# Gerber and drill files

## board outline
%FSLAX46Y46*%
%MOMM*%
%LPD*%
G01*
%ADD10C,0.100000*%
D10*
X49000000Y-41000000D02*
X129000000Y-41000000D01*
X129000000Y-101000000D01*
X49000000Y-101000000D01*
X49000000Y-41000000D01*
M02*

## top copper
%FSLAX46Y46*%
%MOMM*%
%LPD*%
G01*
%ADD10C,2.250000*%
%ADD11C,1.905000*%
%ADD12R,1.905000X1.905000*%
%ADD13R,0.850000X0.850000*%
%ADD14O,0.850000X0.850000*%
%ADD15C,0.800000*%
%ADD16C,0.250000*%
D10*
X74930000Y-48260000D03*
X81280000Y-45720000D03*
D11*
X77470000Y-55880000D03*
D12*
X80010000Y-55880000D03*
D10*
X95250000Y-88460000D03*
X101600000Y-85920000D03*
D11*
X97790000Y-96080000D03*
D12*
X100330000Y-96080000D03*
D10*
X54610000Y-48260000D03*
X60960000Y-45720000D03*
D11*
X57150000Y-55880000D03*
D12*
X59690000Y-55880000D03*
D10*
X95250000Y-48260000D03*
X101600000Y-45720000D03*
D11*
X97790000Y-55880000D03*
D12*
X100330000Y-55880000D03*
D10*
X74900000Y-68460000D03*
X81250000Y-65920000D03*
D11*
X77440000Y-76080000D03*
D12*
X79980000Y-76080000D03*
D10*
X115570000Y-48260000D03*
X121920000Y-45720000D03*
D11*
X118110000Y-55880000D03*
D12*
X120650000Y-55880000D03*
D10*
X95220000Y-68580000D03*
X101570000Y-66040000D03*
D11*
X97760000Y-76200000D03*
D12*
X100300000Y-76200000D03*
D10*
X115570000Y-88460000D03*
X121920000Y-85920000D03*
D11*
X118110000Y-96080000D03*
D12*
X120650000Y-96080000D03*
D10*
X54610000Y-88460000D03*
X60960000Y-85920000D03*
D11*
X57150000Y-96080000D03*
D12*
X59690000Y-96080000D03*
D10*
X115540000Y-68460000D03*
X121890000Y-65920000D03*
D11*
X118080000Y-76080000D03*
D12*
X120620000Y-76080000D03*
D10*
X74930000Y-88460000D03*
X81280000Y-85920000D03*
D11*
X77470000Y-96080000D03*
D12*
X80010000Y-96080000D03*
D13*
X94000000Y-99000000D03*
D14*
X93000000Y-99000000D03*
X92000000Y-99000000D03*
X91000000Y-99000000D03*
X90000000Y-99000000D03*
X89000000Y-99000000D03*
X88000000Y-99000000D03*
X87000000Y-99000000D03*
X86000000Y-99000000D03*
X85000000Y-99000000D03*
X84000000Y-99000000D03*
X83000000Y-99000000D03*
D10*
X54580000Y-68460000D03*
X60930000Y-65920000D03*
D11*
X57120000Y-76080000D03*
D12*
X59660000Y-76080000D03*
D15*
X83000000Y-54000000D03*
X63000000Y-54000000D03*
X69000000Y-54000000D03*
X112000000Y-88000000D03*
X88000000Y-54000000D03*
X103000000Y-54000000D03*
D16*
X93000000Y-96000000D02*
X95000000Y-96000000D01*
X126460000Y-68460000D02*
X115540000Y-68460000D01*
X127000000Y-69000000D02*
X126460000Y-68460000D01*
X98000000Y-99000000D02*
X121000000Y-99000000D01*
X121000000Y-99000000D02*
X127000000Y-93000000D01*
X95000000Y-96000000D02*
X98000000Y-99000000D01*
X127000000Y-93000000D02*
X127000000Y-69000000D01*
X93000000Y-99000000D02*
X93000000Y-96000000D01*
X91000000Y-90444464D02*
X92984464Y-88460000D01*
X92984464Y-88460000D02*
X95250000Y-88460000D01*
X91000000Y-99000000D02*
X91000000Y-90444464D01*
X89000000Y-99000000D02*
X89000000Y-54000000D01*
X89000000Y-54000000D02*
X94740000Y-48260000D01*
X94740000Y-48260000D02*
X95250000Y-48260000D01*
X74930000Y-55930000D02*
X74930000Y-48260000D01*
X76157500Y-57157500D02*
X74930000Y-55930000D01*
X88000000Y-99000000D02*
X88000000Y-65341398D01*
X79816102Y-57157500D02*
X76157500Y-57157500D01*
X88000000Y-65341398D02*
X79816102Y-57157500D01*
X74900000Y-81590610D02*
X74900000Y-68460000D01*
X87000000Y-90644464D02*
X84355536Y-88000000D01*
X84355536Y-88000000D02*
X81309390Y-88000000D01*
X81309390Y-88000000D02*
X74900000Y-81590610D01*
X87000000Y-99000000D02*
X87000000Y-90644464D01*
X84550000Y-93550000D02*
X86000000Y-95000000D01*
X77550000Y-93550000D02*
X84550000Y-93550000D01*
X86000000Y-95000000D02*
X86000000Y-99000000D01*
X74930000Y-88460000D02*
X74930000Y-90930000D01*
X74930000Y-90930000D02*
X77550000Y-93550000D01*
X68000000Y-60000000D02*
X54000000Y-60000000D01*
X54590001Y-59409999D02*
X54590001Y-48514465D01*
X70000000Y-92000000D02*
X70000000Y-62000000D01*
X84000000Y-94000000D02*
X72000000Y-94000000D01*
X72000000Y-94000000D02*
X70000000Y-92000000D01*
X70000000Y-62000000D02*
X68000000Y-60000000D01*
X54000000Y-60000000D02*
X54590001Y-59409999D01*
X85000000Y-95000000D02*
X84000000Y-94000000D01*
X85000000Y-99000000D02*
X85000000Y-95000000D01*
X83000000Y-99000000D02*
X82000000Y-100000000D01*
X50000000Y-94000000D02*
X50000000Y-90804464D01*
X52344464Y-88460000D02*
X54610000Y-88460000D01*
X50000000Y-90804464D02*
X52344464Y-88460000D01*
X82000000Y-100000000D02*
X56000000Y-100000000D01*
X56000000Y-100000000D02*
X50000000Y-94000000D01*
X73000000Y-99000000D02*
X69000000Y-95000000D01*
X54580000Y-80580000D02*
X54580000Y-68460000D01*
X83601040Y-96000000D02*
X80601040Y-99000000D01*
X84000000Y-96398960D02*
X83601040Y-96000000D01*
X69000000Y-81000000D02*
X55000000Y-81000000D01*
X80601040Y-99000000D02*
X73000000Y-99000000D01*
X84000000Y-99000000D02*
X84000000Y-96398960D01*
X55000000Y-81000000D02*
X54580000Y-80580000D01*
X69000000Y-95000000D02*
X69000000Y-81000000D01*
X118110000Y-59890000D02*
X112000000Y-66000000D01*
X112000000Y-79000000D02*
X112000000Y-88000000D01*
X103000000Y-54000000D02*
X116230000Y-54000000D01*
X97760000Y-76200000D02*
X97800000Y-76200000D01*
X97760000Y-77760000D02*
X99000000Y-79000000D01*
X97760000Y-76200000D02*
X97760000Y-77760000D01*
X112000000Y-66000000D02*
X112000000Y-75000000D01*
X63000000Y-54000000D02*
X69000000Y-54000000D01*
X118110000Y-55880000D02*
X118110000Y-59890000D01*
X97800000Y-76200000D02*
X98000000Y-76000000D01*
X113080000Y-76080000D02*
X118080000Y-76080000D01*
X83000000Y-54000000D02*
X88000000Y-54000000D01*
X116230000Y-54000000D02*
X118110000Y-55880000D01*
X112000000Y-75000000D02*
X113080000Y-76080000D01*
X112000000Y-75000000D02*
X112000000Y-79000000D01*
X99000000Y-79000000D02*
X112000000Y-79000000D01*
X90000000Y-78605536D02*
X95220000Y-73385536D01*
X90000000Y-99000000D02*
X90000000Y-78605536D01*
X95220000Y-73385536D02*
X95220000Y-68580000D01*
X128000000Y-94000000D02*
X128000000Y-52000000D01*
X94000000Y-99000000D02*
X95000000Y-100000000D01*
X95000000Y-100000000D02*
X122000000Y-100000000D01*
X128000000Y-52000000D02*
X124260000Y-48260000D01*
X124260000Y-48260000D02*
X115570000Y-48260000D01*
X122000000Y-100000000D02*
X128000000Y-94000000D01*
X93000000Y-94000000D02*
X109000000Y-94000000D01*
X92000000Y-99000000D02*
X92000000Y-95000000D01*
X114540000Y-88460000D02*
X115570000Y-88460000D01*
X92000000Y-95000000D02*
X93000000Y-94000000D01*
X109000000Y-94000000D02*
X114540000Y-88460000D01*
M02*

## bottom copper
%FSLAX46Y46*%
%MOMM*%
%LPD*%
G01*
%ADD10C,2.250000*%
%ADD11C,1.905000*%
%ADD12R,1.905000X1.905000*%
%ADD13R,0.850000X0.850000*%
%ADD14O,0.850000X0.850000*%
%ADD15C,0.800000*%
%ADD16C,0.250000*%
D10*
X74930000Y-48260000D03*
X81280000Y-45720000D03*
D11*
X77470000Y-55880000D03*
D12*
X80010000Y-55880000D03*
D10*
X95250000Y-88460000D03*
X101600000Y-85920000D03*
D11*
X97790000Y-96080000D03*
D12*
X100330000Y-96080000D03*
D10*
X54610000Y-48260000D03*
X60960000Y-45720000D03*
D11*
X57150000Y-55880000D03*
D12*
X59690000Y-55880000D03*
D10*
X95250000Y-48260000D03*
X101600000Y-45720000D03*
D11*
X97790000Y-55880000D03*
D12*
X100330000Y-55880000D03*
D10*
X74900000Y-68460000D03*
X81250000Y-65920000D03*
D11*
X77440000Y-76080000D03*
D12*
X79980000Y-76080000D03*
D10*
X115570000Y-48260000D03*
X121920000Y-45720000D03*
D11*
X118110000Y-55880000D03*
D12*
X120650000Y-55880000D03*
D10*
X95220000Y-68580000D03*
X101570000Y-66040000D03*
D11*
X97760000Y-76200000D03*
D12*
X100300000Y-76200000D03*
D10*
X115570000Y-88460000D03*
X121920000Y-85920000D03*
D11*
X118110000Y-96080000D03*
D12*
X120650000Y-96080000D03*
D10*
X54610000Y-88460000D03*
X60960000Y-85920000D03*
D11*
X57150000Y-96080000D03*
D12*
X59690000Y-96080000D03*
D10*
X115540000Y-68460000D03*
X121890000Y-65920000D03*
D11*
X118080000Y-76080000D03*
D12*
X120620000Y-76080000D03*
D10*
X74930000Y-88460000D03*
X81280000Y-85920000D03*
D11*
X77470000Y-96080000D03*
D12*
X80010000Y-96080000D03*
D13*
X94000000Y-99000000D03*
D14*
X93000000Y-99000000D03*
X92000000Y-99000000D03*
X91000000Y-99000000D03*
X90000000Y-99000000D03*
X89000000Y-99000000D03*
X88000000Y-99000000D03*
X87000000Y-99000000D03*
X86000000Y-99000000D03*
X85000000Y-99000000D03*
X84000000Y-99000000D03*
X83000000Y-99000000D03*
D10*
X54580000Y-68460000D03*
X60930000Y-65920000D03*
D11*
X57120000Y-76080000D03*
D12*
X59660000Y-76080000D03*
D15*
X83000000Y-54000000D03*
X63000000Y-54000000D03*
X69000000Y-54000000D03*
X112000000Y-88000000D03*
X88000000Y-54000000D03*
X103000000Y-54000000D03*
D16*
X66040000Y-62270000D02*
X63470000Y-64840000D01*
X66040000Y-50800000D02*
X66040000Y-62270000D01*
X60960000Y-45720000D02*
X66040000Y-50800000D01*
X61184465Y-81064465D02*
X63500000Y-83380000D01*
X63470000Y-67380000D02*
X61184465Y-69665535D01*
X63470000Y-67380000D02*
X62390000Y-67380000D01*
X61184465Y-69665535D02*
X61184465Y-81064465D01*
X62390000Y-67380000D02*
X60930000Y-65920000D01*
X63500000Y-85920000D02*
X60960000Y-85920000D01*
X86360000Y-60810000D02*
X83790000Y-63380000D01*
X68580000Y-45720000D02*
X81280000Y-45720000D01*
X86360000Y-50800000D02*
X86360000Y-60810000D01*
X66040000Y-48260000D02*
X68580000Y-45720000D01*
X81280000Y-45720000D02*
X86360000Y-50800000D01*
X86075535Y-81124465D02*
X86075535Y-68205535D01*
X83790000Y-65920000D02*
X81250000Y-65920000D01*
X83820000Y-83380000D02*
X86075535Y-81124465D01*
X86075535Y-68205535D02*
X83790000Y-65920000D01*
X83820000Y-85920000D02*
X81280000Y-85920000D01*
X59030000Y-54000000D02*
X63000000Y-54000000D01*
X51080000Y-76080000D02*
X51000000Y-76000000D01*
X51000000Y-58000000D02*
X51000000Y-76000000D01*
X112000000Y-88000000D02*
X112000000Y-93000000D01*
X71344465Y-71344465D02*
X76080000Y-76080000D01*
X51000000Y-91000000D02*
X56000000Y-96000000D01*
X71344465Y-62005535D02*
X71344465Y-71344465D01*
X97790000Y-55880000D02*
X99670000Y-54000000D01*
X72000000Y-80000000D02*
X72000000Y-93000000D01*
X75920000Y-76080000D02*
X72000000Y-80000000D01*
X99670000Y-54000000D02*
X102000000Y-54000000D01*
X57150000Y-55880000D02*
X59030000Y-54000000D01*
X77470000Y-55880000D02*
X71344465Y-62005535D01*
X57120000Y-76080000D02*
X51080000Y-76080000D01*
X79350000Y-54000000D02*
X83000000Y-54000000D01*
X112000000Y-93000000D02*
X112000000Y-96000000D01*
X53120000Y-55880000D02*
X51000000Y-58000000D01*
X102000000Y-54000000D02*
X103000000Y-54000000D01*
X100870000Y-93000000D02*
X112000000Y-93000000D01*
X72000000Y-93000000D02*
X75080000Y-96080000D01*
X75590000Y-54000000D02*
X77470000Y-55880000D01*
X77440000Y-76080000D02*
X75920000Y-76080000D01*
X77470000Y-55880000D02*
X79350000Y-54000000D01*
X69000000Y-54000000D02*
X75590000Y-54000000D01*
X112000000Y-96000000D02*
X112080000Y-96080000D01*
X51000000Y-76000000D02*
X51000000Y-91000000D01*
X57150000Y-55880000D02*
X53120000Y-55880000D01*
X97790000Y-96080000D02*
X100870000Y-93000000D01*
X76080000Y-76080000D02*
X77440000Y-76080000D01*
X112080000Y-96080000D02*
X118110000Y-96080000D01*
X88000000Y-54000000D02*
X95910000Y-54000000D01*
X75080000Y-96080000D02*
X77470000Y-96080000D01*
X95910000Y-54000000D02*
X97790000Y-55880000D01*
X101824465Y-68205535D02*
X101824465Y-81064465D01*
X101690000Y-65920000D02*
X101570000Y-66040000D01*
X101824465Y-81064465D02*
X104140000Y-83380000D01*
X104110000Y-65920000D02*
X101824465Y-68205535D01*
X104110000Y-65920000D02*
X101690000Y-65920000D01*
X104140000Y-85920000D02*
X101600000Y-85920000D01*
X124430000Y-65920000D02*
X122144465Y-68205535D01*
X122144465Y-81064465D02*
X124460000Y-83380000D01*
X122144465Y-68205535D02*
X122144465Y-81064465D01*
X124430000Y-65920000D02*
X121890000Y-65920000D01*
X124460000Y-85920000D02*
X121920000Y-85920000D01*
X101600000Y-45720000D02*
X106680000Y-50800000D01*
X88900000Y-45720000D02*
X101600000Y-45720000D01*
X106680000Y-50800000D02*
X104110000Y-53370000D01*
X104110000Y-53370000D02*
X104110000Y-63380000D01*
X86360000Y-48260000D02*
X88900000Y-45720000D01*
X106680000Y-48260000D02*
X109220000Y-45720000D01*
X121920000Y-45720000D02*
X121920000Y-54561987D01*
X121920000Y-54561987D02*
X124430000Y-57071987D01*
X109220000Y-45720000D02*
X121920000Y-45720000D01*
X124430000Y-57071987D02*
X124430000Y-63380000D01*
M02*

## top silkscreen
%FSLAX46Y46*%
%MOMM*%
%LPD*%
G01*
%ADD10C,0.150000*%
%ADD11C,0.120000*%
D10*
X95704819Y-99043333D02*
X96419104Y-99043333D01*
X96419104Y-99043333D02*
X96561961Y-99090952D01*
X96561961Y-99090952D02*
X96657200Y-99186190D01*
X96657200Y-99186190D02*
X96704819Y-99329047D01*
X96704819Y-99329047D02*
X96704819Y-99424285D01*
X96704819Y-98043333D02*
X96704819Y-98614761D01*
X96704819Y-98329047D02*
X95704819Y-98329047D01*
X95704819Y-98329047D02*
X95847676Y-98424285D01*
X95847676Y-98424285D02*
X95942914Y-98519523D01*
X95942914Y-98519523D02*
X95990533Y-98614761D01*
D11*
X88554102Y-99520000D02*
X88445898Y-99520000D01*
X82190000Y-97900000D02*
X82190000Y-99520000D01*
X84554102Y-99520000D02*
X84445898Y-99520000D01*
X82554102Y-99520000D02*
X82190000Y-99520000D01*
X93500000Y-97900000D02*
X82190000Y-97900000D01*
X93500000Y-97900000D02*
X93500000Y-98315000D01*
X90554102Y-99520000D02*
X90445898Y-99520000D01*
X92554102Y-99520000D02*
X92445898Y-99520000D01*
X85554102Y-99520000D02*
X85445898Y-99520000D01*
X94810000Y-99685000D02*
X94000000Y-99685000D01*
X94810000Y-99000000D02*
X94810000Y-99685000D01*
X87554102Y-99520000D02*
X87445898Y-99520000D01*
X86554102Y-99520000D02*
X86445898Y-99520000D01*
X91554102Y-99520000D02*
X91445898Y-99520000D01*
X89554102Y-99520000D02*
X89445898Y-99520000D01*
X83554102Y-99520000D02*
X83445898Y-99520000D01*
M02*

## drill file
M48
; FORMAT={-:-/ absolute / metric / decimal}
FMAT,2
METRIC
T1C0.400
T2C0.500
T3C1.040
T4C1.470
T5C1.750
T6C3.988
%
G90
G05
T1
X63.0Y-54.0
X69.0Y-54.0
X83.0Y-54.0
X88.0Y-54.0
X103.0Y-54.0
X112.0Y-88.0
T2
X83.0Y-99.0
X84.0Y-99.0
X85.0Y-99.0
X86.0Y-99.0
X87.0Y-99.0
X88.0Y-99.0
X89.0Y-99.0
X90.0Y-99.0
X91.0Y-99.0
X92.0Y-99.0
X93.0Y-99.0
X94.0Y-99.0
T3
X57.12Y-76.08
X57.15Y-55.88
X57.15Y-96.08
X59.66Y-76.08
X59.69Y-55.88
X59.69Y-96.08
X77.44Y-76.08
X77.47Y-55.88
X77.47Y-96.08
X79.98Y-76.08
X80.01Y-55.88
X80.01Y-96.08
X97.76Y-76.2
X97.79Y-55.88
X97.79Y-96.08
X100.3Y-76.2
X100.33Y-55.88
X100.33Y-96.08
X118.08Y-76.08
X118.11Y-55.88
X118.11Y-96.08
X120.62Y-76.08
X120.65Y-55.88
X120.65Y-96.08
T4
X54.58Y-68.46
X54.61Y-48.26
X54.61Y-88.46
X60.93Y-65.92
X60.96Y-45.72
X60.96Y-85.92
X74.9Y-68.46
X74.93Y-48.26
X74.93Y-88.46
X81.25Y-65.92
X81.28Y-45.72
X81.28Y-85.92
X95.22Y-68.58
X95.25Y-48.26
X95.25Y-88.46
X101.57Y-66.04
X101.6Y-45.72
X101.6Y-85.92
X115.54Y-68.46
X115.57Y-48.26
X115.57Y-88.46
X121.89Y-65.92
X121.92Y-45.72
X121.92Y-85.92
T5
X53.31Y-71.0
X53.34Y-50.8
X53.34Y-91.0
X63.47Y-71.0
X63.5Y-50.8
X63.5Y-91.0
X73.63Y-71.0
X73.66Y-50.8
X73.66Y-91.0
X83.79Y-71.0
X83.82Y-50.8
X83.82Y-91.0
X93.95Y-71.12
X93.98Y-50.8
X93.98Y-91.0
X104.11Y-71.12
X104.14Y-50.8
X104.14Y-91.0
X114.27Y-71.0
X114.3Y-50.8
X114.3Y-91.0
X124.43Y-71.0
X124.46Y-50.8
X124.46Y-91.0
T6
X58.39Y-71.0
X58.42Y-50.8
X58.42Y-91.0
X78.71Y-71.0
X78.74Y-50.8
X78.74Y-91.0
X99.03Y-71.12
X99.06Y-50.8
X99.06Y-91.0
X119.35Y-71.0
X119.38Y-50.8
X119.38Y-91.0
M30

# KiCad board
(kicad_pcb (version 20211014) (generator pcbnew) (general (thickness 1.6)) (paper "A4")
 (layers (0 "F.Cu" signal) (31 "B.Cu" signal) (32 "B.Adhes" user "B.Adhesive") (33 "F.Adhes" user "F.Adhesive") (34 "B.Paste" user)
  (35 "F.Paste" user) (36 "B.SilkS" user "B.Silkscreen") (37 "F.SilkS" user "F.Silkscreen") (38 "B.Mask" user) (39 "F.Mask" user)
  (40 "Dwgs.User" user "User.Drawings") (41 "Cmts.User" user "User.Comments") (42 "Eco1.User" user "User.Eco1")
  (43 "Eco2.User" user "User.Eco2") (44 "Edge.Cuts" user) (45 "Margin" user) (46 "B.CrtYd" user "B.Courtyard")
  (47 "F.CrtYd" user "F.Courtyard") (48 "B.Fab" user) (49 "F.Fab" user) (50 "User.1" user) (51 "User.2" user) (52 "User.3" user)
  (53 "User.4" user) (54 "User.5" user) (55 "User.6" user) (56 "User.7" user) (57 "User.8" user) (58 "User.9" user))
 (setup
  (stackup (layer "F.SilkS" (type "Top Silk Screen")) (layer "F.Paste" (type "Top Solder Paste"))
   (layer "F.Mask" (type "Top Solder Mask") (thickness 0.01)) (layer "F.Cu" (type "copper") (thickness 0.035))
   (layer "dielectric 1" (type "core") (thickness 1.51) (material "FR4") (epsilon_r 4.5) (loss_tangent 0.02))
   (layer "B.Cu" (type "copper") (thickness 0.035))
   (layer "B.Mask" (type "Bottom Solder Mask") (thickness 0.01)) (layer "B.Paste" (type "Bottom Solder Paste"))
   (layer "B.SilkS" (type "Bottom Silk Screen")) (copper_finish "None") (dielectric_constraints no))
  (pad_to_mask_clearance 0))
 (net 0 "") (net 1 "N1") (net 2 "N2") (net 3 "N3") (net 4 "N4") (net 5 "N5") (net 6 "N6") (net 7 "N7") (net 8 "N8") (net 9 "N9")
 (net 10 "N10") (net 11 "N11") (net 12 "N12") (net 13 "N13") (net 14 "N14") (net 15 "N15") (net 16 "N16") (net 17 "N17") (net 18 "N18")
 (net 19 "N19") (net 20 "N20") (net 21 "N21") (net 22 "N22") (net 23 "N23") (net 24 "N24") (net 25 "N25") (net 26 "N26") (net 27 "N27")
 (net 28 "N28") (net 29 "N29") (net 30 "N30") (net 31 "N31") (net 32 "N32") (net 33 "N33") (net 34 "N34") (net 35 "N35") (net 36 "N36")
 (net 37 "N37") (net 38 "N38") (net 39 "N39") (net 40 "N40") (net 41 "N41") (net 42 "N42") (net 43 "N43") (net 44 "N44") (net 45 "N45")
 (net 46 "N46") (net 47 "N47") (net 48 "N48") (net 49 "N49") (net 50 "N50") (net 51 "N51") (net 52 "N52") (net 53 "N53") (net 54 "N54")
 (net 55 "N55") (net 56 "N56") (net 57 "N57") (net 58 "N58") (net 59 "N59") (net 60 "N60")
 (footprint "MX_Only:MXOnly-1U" (layer "F.Cu") (at 78.74 50.8)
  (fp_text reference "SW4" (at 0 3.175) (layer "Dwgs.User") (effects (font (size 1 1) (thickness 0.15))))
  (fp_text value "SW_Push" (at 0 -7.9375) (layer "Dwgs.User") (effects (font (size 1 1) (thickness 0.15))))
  (pad "" np_thru_hole circle locked (at -5.08 0 48.0996) (size 1.75 1.75) (drill 1.75) (layers *.Cu *.Mask))
  (pad "" np_thru_hole circle locked (at 0 0) (size 3.9878 3.9878) (drill 3.9878) (layers *.Cu *.Mask))
  (pad "" np_thru_hole circle locked (at 5.08 0 48.0996) (size 1.75 1.75) (drill 1.75) (layers *.Cu *.Mask))
  (pad "1" thru_hole circle locked (at -3.81 -2.54) (size 2.25 2.25) (drill 1.47) (layers *.Cu "B.Mask") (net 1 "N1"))
  (pad "2" thru_hole circle locked (at 2.54 -5.08) (size 2.25 2.25) (drill 1.47) (layers *.Cu "B.Mask") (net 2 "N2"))
  (pad "3" thru_hole circle locked (at -1.27 5.08) (size 1.905 1.905) (drill 1.04) (layers *.Cu "B.Mask") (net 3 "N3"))
  (pad "4" thru_hole rect locked (at 1.27 5.08) (size 1.905 1.905) (drill 1.04) (layers *.Cu "B.Mask") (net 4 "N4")))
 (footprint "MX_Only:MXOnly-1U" (layer "F.Cu") (at 99.06 91)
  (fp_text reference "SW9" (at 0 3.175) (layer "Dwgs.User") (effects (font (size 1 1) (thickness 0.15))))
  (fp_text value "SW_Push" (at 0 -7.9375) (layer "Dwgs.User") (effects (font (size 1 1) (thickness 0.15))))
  (pad "" np_thru_hole circle locked (at -5.08 0 48.0996) (size 1.75 1.75) (drill 1.75) (layers *.Cu *.Mask))
  (pad "" np_thru_hole circle locked (at 5.08 0 48.0996) (size 1.75 1.75) (drill 1.75) (layers *.Cu *.Mask))
  (pad "" np_thru_hole circle locked (at 0 0) (size 3.9878 3.9878) (drill 3.9878) (layers *.Cu *.Mask))
  (pad "1" thru_hole circle locked (at -3.81 -2.54) (size 2.25 2.25) (drill 1.47) (layers *.Cu "B.Mask") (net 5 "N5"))
  (pad "2" thru_hole circle locked (at 2.54 -5.08) (size 2.25 2.25) (drill 1.47) (layers *.Cu "B.Mask") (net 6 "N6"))
  (pad "3" thru_hole circle locked (at -1.27 5.08) (size 1.905 1.905) (drill 1.04) (layers *.Cu "B.Mask") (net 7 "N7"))
  (pad "4" thru_hole rect locked (at 1.27 5.08) (size 1.905 1.905) (drill 1.04) (layers *.Cu "B.Mask") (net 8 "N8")))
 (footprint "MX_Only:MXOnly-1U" (layer "F.Cu") (at 58.42 50.8)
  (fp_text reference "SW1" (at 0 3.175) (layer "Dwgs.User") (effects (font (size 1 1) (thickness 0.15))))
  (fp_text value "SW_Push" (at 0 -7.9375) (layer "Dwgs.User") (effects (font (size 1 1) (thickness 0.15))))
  (pad "" np_thru_hole circle locked (at 5.08 0 48.0996) (size 1.75 1.75) (drill 1.75) (layers *.Cu *.Mask))
  (pad "" np_thru_hole circle locked (at -5.08 0 48.0996) (size 1.75 1.75) (drill 1.75) (layers *.Cu *.Mask))
  (pad "" np_thru_hole circle locked (at 0 0) (size 3.9878 3.9878) (drill 3.9878) (layers *.Cu *.Mask))
  (pad "1" thru_hole circle locked (at -3.81 -2.54) (size 2.25 2.25) (drill 1.47) (layers *.Cu "B.Mask") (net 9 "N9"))
  (pad "2" thru_hole circle locked (at 2.54 -5.08) (size 2.25 2.25) (drill 1.47) (layers *.Cu "B.Mask") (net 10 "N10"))
  (pad "3" thru_hole circle locked (at -1.27 5.08) (size 1.905 1.905) (drill 1.04) (layers *.Cu "B.Mask") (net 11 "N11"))
  (pad "4" thru_hole rect locked (at 1.27 5.08) (size 1.905 1.905) (drill 1.04) (layers *.Cu "B.Mask") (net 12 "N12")))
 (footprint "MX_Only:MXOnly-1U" (layer "F.Cu") (at 99.06 50.8)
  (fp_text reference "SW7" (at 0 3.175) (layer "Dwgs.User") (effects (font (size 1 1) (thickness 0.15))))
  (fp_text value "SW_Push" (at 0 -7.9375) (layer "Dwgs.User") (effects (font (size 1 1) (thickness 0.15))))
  (pad "" np_thru_hole circle locked (at 0 0) (size 3.9878 3.9878) (drill 3.9878) (layers *.Cu *.Mask))
  (pad "" np_thru_hole circle locked (at -5.08 0 48.0996) (size 1.75 1.75) (drill 1.75) (layers *.Cu *.Mask))
  (pad "" np_thru_hole circle locked (at 5.08 0 48.0996) (size 1.75 1.75) (drill 1.75) (layers *.Cu *.Mask))
  (pad "1" thru_hole circle locked (at -3.81 -2.54) (size 2.25 2.25) (drill 1.47) (layers *.Cu "B.Mask") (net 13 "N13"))
  (pad "2" thru_hole circle locked (at 2.54 -5.08) (size 2.25 2.25) (drill 1.47) (layers *.Cu "B.Mask") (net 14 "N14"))
  (pad "3" thru_hole circle locked (at -1.27 5.08) (size 1.905 1.905) (drill 1.04) (layers *.Cu "B.Mask") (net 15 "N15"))
  (pad "4" thru_hole rect locked (at 1.27 5.08) (size 1.905 1.905) (drill 1.04) (layers *.Cu "B.Mask") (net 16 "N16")))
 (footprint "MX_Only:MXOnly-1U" (layer "F.Cu") (at 78.71 71)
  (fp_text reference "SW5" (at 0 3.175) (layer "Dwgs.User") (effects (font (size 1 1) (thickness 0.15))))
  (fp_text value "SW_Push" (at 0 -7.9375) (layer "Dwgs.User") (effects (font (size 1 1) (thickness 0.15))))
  (pad "" np_thru_hole circle locked (at -5.08 0 48.0996) (size 1.75 1.75) (drill 1.75) (layers *.Cu *.Mask))
  (pad "" np_thru_hole circle locked (at 5.08 0 48.0996) (size 1.75 1.75) (drill 1.75) (layers *.Cu *.Mask))
  (pad "" np_thru_hole circle locked (at 0 0) (size 3.9878 3.9878) (drill 3.9878) (layers *.Cu *.Mask))
  (pad "1" thru_hole circle locked (at -3.81 -2.54) (size 2.25 2.25) (drill 1.47) (layers *.Cu "B.Mask") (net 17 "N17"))
  (pad "2" thru_hole circle locked (at 2.54 -5.08) (size 2.25 2.25) (drill 1.47) (layers *.Cu "B.Mask") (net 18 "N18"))
  (pad "3" thru_hole circle locked (at -1.27 5.08) (size 1.905 1.905) (drill 1.04) (layers *.Cu "B.Mask") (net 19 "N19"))
  (pad "4" thru_hole rect locked (at 1.27 5.08) (size 1.905 1.905) (drill 1.04) (layers *.Cu "B.Mask") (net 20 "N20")))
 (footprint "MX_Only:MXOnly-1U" (layer "F.Cu") (at 119.38 50.8)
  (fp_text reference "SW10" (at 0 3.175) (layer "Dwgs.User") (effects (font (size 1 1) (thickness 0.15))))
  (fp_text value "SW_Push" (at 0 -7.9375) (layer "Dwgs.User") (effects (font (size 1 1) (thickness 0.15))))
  (pad "" np_thru_hole circle locked (at 0 0) (size 3.9878 3.9878) (drill 3.9878) (layers *.Cu *.Mask))
  (pad "" np_thru_hole circle locked (at 5.08 0 48.0996) (size 1.75 1.75) (drill 1.75) (layers *.Cu *.Mask))
  (pad "" np_thru_hole circle locked (at -5.08 0 48.0996) (size 1.75 1.75) (drill 1.75) (layers *.Cu *.Mask))
  (pad "1" thru_hole circle locked (at -3.81 -2.54) (size 2.25 2.25) (drill 1.47) (layers *.Cu "B.Mask") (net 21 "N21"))
  (pad "2" thru_hole circle locked (at 2.54 -5.08) (size 2.25 2.25) (drill 1.47) (layers *.Cu "B.Mask") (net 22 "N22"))
  (pad "3" thru_hole circle locked (at -1.27 5.08) (size 1.905 1.905) (drill 1.04) (layers *.Cu "B.Mask") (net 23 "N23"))
  (pad "4" thru_hole rect locked (at 1.27 5.08) (size 1.905 1.905) (drill 1.04) (layers *.Cu "B.Mask") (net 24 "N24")))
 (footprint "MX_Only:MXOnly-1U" (layer "F.Cu") (at 99.03 71.12)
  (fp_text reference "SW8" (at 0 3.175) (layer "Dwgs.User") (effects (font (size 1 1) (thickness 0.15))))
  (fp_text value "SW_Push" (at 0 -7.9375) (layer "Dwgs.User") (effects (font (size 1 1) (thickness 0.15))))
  (pad "" np_thru_hole circle locked (at 0 0) (size 3.9878 3.9878) (drill 3.9878) (layers *.Cu *.Mask))
  (pad "" np_thru_hole circle locked (at 5.08 0 48.0996) (size 1.75 1.75) (drill 1.75) (layers *.Cu *.Mask))
  (pad "" np_thru_hole circle locked (at -5.08 0 48.0996) (size 1.75 1.75) (drill 1.75) (layers *.Cu *.Mask))
  (pad "1" thru_hole circle locked (at -3.81 -2.54) (size 2.25 2.25) (drill 1.47) (layers *.Cu "B.Mask") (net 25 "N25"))
  (pad "2" thru_hole circle locked (at 2.54 -5.08) (size 2.25 2.25) (drill 1.47) (layers *.Cu "B.Mask") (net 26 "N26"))
  (pad "3" thru_hole circle locked (at -1.27 5.08) (size 1.905 1.905) (drill 1.04) (layers *.Cu "B.Mask") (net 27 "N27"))
  (pad "4" thru_hole rect locked (at 1.27 5.08) (size 1.905 1.905) (drill 1.04) (layers *.Cu "B.Mask") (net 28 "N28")))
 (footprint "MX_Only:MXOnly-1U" (layer "F.Cu") (at 119.38 91)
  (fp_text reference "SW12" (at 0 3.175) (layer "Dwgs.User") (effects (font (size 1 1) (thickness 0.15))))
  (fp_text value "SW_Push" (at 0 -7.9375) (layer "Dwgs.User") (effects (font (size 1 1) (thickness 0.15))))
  (pad "" np_thru_hole circle locked (at 0 0) (size 3.9878 3.9878) (drill 3.9878) (layers *.Cu *.Mask))
  (pad "" np_thru_hole circle locked (at 5.08 0 48.0996) (size 1.75 1.75) (drill 1.75) (layers *.Cu *.Mask))
  (pad "" np_thru_hole circle locked (at -5.08 0 48.0996) (size 1.75 1.75) (drill 1.75) (layers *.Cu *.Mask))
  (pad "1" thru_hole circle locked (at -3.81 -2.54) (size 2.25 2.25) (drill 1.47) (layers *.Cu "B.Mask") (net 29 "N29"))
  (pad "2" thru_hole circle locked (at 2.54 -5.08) (size 2.25 2.25) (drill 1.47) (layers *.Cu "B.Mask") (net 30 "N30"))
  (pad "3" thru_hole circle locked (at -1.27 5.08) (size 1.905 1.905) (drill 1.04) (layers *.Cu "B.Mask") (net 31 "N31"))
  (pad "4" thru_hole rect locked (at 1.27 5.08) (size 1.905 1.905) (drill 1.04) (layers *.Cu "B.Mask") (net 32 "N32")))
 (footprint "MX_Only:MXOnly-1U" (layer "F.Cu") (at 58.42 91)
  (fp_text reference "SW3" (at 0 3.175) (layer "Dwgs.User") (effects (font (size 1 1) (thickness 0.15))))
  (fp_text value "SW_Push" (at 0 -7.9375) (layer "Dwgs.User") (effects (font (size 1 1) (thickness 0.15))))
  (pad "" np_thru_hole circle locked (at -5.08 0 48.0996) (size 1.75 1.75) (drill 1.75) (layers *.Cu *.Mask))
  (pad "" np_thru_hole circle locked (at 5.08 0 48.0996) (size 1.75 1.75) (drill 1.75) (layers *.Cu *.Mask))
  (pad "" np_thru_hole circle locked (at 0 0) (size 3.9878 3.9878) (drill 3.9878) (layers *.Cu *.Mask))
  (pad "1" thru_hole circle locked (at -3.81 -2.54) (size 2.25 2.25) (drill 1.47) (layers *.Cu "B.Mask") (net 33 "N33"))
  (pad "2" thru_hole circle locked (at 2.54 -5.08) (size 2.25 2.25) (drill 1.47) (layers *.Cu "B.Mask") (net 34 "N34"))
  (pad "3" thru_hole circle locked (at -1.27 5.08) (size 1.905 1.905) (drill 1.04) (layers *.Cu "B.Mask") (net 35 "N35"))
  (pad "4" thru_hole rect locked (at 1.27 5.08) (size 1.905 1.905) (drill 1.04) (layers *.Cu "B.Mask") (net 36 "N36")))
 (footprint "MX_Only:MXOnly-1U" (layer "F.Cu") (at 119.35 71)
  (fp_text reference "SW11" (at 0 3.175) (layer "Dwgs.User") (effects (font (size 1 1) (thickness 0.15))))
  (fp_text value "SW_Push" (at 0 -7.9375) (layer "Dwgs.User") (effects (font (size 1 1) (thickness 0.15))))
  (pad "" np_thru_hole circle locked (at -5.08 0 48.0996) (size 1.75 1.75) (drill 1.75) (layers *.Cu *.Mask))
  (pad "" np_thru_hole circle locked (at 5.08 0 48.0996) (size 1.75 1.75) (drill 1.75) (layers *.Cu *.Mask))
  (pad "" np_thru_hole circle locked (at 0 0) (size 3.9878 3.9878) (drill 3.9878) (layers *.Cu *.Mask))
  (pad "1" thru_hole circle locked (at -3.81 -2.54) (size 2.25 2.25) (drill 1.47) (layers *.Cu "B.Mask") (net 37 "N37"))
  (pad "2" thru_hole circle locked (at 2.54 -5.08) (size 2.25 2.25) (drill 1.47) (layers *.Cu "B.Mask") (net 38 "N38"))
  (pad "3" thru_hole circle locked (at -1.27 5.08) (size 1.905 1.905) (drill 1.04) (layers *.Cu "B.Mask") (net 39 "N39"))
  (pad "4" thru_hole rect locked (at 1.27 5.08) (size 1.905 1.905) (drill 1.04) (layers *.Cu "B.Mask") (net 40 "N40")))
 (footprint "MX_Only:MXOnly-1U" (layer "F.Cu") (at 78.74 91)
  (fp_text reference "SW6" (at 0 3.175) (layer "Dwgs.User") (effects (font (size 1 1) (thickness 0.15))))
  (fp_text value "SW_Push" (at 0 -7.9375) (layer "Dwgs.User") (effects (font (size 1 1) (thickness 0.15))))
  (pad "" np_thru_hole circle locked (at 0 0) (size 3.9878 3.9878) (drill 3.9878) (layers *.Cu *.Mask))
  (pad "" np_thru_hole circle locked (at -5.08 0 48.0996) (size 1.75 1.75) (drill 1.75) (layers *.Cu *.Mask))
  (pad "" np_thru_hole circle locked (at 5.08 0 48.0996) (size 1.75 1.75) (drill 1.75) (layers *.Cu *.Mask))
  (pad "1" thru_hole circle locked (at -3.81 -2.54) (size 2.25 2.25) (drill 1.47) (layers *.Cu "B.Mask") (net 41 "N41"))
  (pad "2" thru_hole circle locked (at 2.54 -5.08) (size 2.25 2.25) (drill 1.47) (layers *.Cu "B.Mask") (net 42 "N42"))
  (pad "3" thru_hole circle locked (at -1.27 5.08) (size 1.905 1.905) (drill 1.04) (layers *.Cu "B.Mask") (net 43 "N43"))
  (pad "4" thru_hole rect locked (at 1.27 5.08) (size 1.905 1.905) (drill 1.04) (layers *.Cu "B.Mask") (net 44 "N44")))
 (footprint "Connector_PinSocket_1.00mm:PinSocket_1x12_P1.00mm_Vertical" (layer "F.Cu") (at 94 99 -90)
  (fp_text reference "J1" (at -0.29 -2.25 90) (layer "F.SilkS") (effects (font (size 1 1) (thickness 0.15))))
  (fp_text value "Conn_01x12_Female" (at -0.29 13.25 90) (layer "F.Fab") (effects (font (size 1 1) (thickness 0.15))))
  (fp_line (start 0.52 5.445898) (end 0.52 5.554102) (layer "F.SilkS") (width 0.12))
  (fp_line (start -1.1 11.81) (end 0.52 11.81) (layer "F.SilkS") (width 0.12))
  (fp_line (start 0.52 9.445898) (end 0.52 9.554102) (layer "F.SilkS") (width 0.12))
  (fp_line (start 0.52 11.445898) (end 0.52 11.81) (layer "F.SilkS") (width 0.12))
  (fp_line (start -1.1 0.5) (end -1.1 11.81) (layer "F.SilkS") (width 0.12))
  (fp_line (start -1.1 0.5) (end -0.685 0.5) (layer "F.SilkS") (width 0.12))
  (fp_line (start 0.52 3.445898) (end 0.52 3.554102) (layer "F.SilkS") (width 0.12))
  (fp_line (start 0.52 1.445898) (end 0.52 1.554102) (layer "F.SilkS") (width 0.12))
  (fp_line (start 0.52 8.445898) (end 0.52 8.554102) (layer "F.SilkS") (width 0.12))
  (fp_line (start 0.685 -0.81) (end 0.685 0) (layer "F.SilkS") (width 0.12))
  (fp_line (start 0 -0.81) (end 0.685 -0.81) (layer "F.SilkS") (width 0.12))
  (fp_line (start 0.52 6.445898) (end 0.52 6.554102) (layer "F.SilkS") (width 0.12))
  (fp_line (start 0.52 7.445898) (end 0.52 7.554102) (layer "F.SilkS") (width 0.12))
  (fp_line (start 0.52 2.445898) (end 0.52 2.554102) (layer "F.SilkS") (width 0.12))
  (fp_line (start 0.52 4.445898) (end 0.52 4.554102) (layer "F.SilkS") (width 0.12))
  (fp_line (start 0.52 10.445898) (end 0.52 10.554102) (layer "F.SilkS") (width 0.12))
  (pad "1" thru_hole rect (at 0 0 270) (size 0.85 0.85) (drill 0.5) (layers *.Cu *.Mask) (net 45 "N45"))
  (pad "2" thru_hole oval (at 0 1 270) (size 0.85 0.85) (drill 0.5) (layers *.Cu *.Mask) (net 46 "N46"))
  (pad "3" thru_hole oval (at 0 2 270) (size 0.85 0.85) (drill 0.5) (layers *.Cu *.Mask) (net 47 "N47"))
  (pad "4" thru_hole oval (at 0 3 270) (size 0.85 0.85) (drill 0.5) (layers *.Cu *.Mask) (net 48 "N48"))
  (pad "5" thru_hole oval (at 0 4 270) (size 0.85 0.85) (drill 0.5) (layers *.Cu *.Mask) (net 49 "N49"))
  (pad "6" thru_hole oval (at 0 5 270) (size 0.85 0.85) (drill 0.5) (layers *.Cu *.Mask) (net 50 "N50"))
  (pad "7" thru_hole oval (at 0 6 270) (size 0.85 0.85) (drill 0.5) (layers *.Cu *.Mask) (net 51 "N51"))
  (pad "8" thru_hole oval (at 0 7 270) (size 0.85 0.85) (drill 0.5) (layers *.Cu *.Mask) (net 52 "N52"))
  (pad "9" thru_hole oval (at 0 8 270) (size 0.85 0.85) (drill 0.5) (layers *.Cu *.Mask) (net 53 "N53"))
  (pad "10" thru_hole oval (at 0 9 270) (size 0.85 0.85) (drill 0.5) (layers *.Cu *.Mask) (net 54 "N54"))
  (pad "11" thru_hole oval (at 0 10 270) (size 0.85 0.85) (drill 0.5) (layers *.Cu *.Mask) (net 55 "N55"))
  (pad "12" thru_hole oval (at 0 11 270) (size 0.85 0.85) (drill 0.5) (layers *.Cu *.Mask) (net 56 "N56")))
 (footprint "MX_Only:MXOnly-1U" (layer "F.Cu") (at 58.39 71)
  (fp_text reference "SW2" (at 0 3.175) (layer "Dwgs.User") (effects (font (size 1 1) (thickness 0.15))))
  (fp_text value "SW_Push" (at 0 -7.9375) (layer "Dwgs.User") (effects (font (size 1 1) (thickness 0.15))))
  (pad "" np_thru_hole circle locked (at 5.08 0 48.0996) (size 1.75 1.75) (drill 1.75) (layers *.Cu *.Mask))
  (pad "" np_thru_hole circle locked (at 0 0) (size 3.9878 3.9878) (drill 3.9878) (layers *.Cu *.Mask))
  (pad "" np_thru_hole circle locked (at -5.08 0 48.0996) (size 1.75 1.75) (drill 1.75) (layers *.Cu *.Mask))
  (pad "1" thru_hole circle locked (at -3.81 -2.54) (size 2.25 2.25) (drill 1.47) (layers *.Cu "B.Mask") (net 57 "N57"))
  (pad "2" thru_hole circle locked (at 2.54 -5.08) (size 2.25 2.25) (drill 1.47) (layers *.Cu "B.Mask") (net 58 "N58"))
  (pad "3" thru_hole circle locked (at -1.27 5.08) (size 1.905 1.905) (drill 1.04) (layers *.Cu "B.Mask") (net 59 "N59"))
  (pad "4" thru_hole rect locked (at 1.27 5.08) (size 1.905 1.905) (drill 1.04) (layers *.Cu "B.Mask") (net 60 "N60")))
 (gr_rect (start 49 41) (end 129 101) (layer "Edge.Cuts") (width 0.1) (fill none))
 (segment (start 93 96) (end 95 96) (width 0.25) (layer "F.Cu") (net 46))
 (segment (start 126.46 68.46) (end 115.54 68.46) (width 0.25) (layer "F.Cu") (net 46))
 (segment (start 127 69) (end 126.46 68.46) (width 0.25) (layer "F.Cu") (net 46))
 (segment (start 98 99) (end 121 99) (width 0.25) (layer "F.Cu") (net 46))
 (segment (start 121 99) (end 127 93) (width 0.25) (layer "F.Cu") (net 46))
 (segment (start 95 96) (end 98 99) (width 0.25) (layer "F.Cu") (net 46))
 (segment (start 127 93) (end 127 69) (width 0.25) (layer "F.Cu") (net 46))
 (segment (start 93 99) (end 93 96) (width 0.25) (layer "F.Cu") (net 46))
 (segment (start 91 90.444464) (end 92.984464 88.46) (width 0.25) (layer "F.Cu") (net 48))
 (segment (start 92.984464 88.46) (end 95.25 88.46) (width 0.25) (layer "F.Cu") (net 48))
 (segment (start 91 99) (end 91 90.444464) (width 0.25) (layer "F.Cu") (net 48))
 (segment (start 89 99) (end 89 54) (width 0.25) (layer "F.Cu") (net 50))
 (segment (start 89 54) (end 94.74 48.26) (width 0.25) (layer "F.Cu") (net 50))
 (segment (start 94.74 48.26) (end 95.25 48.26) (width 0.25) (layer "F.Cu") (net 50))
 (segment (start 74.93 55.93) (end 74.93 48.26) (width 0.25) (layer "F.Cu") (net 51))
 (segment (start 76.1575 57.1575) (end 74.93 55.93) (width 0.25) (layer "F.Cu") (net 51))
 (segment (start 88 99) (end 88 65.341398) (width 0.25) (layer "F.Cu") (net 51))
 (segment (start 79.816102 57.1575) (end 76.1575 57.1575) (width 0.25) (layer "F.Cu") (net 51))
 (segment (start 88 65.341398) (end 79.816102 57.1575) (width 0.25) (layer "F.Cu") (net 51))
 (segment (start 74.9 81.59061) (end 74.9 68.46) (width 0.25) (layer "F.Cu") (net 52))
 (segment (start 87 90.644464) (end 84.355536 88) (width 0.25) (layer "F.Cu") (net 52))
 (segment (start 84.355536 88) (end 81.30939 88) (width 0.25) (layer "F.Cu") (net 52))
 (segment (start 81.30939 88) (end 74.9 81.59061) (width 0.25) (layer "F.Cu") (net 52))
 (segment (start 87 99) (end 87 90.644464) (width 0.25) (layer "F.Cu") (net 52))
 (segment (start 84.55 93.55) (end 86 95) (width 0.25) (layer "F.Cu") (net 53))
 (segment (start 77.55 93.55) (end 84.55 93.55) (width 0.25) (layer "F.Cu") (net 53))
 (segment (start 86 95) (end 86 99) (width 0.25) (layer "F.Cu") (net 53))
 (segment (start 74.93 88.46) (end 74.93 90.93) (width 0.25) (layer "F.Cu") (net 53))
 (segment (start 74.93 90.93) (end 77.55 93.55) (width 0.25) (layer "F.Cu") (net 53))
 (segment (start 68 60) (end 54 60) (width 0.25) (layer "F.Cu") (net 54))
 (segment (start 54.590001 59.409999) (end 54.590001 48.514465) (width 0.25) (layer "F.Cu") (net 54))
 (segment (start 70 92) (end 70 62) (width 0.25) (layer "F.Cu") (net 54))
 (segment (start 84 94) (end 72 94) (width 0.25) (layer "F.Cu") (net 54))
 (segment (start 72 94) (end 70 92) (width 0.25) (layer "F.Cu") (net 54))
 (segment (start 70 62) (end 68 60) (width 0.25) (layer "F.Cu") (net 54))
 (segment (start 54 60) (end 54.590001 59.409999) (width 0.25) (layer "F.Cu") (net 54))
 (segment (start 85 95) (end 84 94) (width 0.25) (layer "F.Cu") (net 54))
 (segment (start 85 99) (end 85 95) (width 0.25) (layer "F.Cu") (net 54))
 (segment (start 83 99) (end 82 100) (width 0.25) (layer "F.Cu") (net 56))
 (segment (start 50 94) (end 50 90.804464) (width 0.25) (layer "F.Cu") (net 56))
 (segment (start 52.344464 88.46) (end 54.61 88.46) (width 0.25) (layer "F.Cu") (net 56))
 (segment (start 50 90.804464) (end 52.344464 88.46) (width 0.25) (layer "F.Cu") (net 56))
 (segment (start 82 100) (end 56 100) (width 0.25) (layer "F.Cu") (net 56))
 (segment (start 56 100) (end 50 94) (width 0.25) (layer "F.Cu") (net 56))
 (segment (start 66.04 62.27) (end 63.47 64.84) (width 0.25) (layer "B.Cu") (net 10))
 (segment (start 66.04 50.8) (end 66.04 62.27) (width 0.25) (layer "B.Cu") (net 10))
 (segment (start 60.96 45.72) (end 66.04 50.8) (width 0.25) (layer "B.Cu") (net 10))
 (segment (start 73 99) (end 69 95) (width 0.25) (layer "F.Cu") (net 57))
 (segment (start 54.58 80.58) (end 54.58 68.46) (width 0.25) (layer "F.Cu") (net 57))
 (segment (start 83.60104 96) (end 80.60104 99) (width 0.25) (layer "F.Cu") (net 57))
 (segment (start 84 96.39896) (end 83.60104 96) (width 0.25) (layer "F.Cu") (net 57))
 (segment (start 69 81) (end 55 81) (width 0.25) (layer "F.Cu") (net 57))
 (segment (start 80.60104 99) (end 73 99) (width 0.25) (layer "F.Cu") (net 57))
 (segment (start 84 99) (end 84 96.39896) (width 0.25) (layer "F.Cu") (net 57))
 (segment (start 55 81) (end 54.58 80.58) (width 0.25) (layer "F.Cu") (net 57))
 (segment (start 69 95) (end 69 81) (width 0.25) (layer "F.Cu") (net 57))
 (segment (start 61.184465 81.064465) (end 63.5 83.38) (width 0.25) (layer "B.Cu") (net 58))
 (segment (start 63.47 67.38) (end 61.184465 69.665535) (width 0.25) (layer "B.Cu") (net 58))
 (segment (start 63.47 67.38) (end 62.39 67.38) (width 0.25) (layer "B.Cu") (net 58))
 (segment (start 61.184465 69.665535) (end 61.184465 81.064465) (width 0.25) (layer "B.Cu") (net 58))
 (segment (start 62.39 67.38) (end 60.93 65.92) (width 0.25) (layer "B.Cu") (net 58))
 (segment (start 63.5 85.92) (end 60.96 85.92) (width 0.25) (layer "B.Cu") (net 34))
 (segment (start 86.36 60.81) (end 83.79 63.38) (width 0.25) (layer "B.Cu") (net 2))
 (segment (start 68.58 45.72) (end 81.28 45.72) (width 0.25) (layer "B.Cu") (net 2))
 (segment (start 86.36 50.8) (end 86.36 60.81) (width 0.25) (layer "B.Cu") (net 2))
 (segment (start 66.04 48.26) (end 68.58 45.72) (width 0.25) (layer "B.Cu") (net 2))
 (segment (start 81.28 45.72) (end 86.36 50.8) (width 0.25) (layer "B.Cu") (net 2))
 (segment (start 86.075535 81.124465) (end 86.075535 68.205535) (width 0.25) (layer "B.Cu") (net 18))
 (segment (start 83.79 65.92) (end 81.25 65.92) (width 0.25) (layer "B.Cu") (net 18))
 (segment (start 83.82 83.38) (end 86.075535 81.124465) (width 0.25) (layer "B.Cu") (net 18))
 (segment (start 86.075535 68.205535) (end 83.79 65.92) (width 0.25) (layer "B.Cu") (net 18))
 (segment (start 83.82 85.92) (end 81.28 85.92) (width 0.25) (layer "B.Cu") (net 42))
 (segment (start 118.11 59.89) (end 112 66) (width 0.25) (layer "F.Cu") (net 43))
 (segment (start 112 79) (end 112 88) (width 0.25) (layer "F.Cu") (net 43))
 (segment (start 103 54) (end 116.23 54) (width 0.25) (layer "F.Cu") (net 43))
 (segment (start 97.76 76.2) (end 97.8 76.2) (width 0.25) (layer "F.Cu") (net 43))
 (segment (start 97.76 77.76) (end 99 79) (width 0.25) (layer "F.Cu") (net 43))
 (segment (start 97.76 76.2) (end 97.76 77.76) (width 0.25) (layer "F.Cu") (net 43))
 (segment (start 112 66) (end 112 75) (width 0.25) (layer "F.Cu") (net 43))
 (segment (start 63 54) (end 69 54) (width 0.25) (layer "F.Cu") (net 43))
 (segment (start 118.11 55.88) (end 118.11 59.89) (width 0.25) (layer "F.Cu") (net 43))
 (segment (start 97.8 76.2) (end 98 76) (width 0.25) (layer "F.Cu") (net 43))
 (segment (start 113.08 76.08) (end 118.08 76.08) (width 0.25) (layer "F.Cu") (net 43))
 (segment (start 83 54) (end 88 54) (width 0.25) (layer "F.Cu") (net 43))
 (segment (start 116.23 54) (end 118.11 55.88) (width 0.25) (layer "F.Cu") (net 43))
 (segment (start 112 75) (end 113.08 76.08) (width 0.25) (layer "F.Cu") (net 43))
 (segment (start 112 75) (end 112 79) (width 0.25) (layer "F.Cu") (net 43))
 (segment (start 99 79) (end 112 79) (width 0.25) (layer "F.Cu") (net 43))
 (via (at 83 54) (size 0.8) (drill 0.4) (layers "F.Cu" "B.Cu") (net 43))
 (via (at 63 54) (size 0.8) (drill 0.4) (layers "F.Cu" "B.Cu") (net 43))
 (via (at 69 54) (size 0.8) (drill 0.4) (layers "F.Cu" "B.Cu") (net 43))
 (via (at 112 88) (size 0.8) (drill 0.4) (layers "F.Cu" "B.Cu") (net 43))
 (via (at 88 54) (size 0.8) (drill 0.4) (layers "F.Cu" "B.Cu") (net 43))
 (via (at 103 54) (size 0.8) (drill 0.4) (layers "F.Cu" "B.Cu") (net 43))
 (segment (start 59.03 54) (end 63 54) (width 0.25) (layer "B.Cu") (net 43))
 (segment (start 51.08 76.08) (end 51 76) (width 0.25) (layer "B.Cu") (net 43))
 (segment (start 51 58) (end 51 76) (width 0.25) (layer "B.Cu") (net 43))
 (segment (start 112 88) (end 112 93) (width 0.25) (layer "B.Cu") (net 43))
 (segment (start 71.344465 71.344465) (end 76.08 76.08) (width 0.25) (layer "B.Cu") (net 43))
 (segment (start 51 91) (end 56 96) (width 0.25) (layer "B.Cu") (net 43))
 (segment (start 71.344465 62.005535) (end 71.344465 71.344465) (width 0.25) (layer "B.Cu") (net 43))
 (segment (start 97.79 55.88) (end 99.67 54) (width 0.25) (layer "B.Cu") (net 43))
 (segment (start 72 80) (end 72 93) (width 0.25) (layer "B.Cu") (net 43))
 (segment (start 75.92 76.08) (end 72 80) (width 0.25) (layer "B.Cu") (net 43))
 (segment (start 99.67 54) (end 102 54) (width 0.25) (layer "B.Cu") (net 43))
 (segment (start 57.15 55.88) (end 59.03 54) (width 0.25) (layer "B.Cu") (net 43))
 (segment (start 77.47 55.88) (end 71.344465 62.005535) (width 0.25) (layer "B.Cu") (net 43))
 (segment (start 57.12 76.08) (end 51.08 76.08) (width 0.25) (layer "B.Cu") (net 43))
 (segment (start 79.35 54) (end 83 54) (width 0.25) (layer "B.Cu") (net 43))
 (segment (start 112 93) (end 112 96) (width 0.25) (layer "B.Cu") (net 43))
 (segment (start 53.12 55.88) (end 51 58) (width 0.25) (layer "B.Cu") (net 43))
 (segment (start 102 54) (end 103 54) (width 0.25) (layer "B.Cu") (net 43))
 (segment (start 100.87 93) (end 112 93) (width 0.25) (layer "B.Cu") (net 43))
 (segment (start 72 93) (end 75.08 96.08) (width 0.25) (layer "B.Cu") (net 43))
 (segment (start 75.59 54) (end 77.47 55.88) (width 0.25) (layer "B.Cu") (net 43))
 (segment (start 77.44 76.08) (end 75.92 76.08) (width 0.25) (layer "B.Cu") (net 43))
 (segment (start 77.47 55.88) (end 79.35 54) (width 0.25) (layer "B.Cu") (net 43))
 (segment (start 69 54) (end 75.59 54) (width 0.25) (layer "B.Cu") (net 43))
 (segment (start 112 96) (end 112.08 96.08) (width 0.25) (layer "B.Cu") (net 43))
 (segment (start 51 76) (end 51 91) (width 0.25) (layer "B.Cu") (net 43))
 (segment (start 57.15 55.88) (end 53.12 55.88) (width 0.25) (layer "B.Cu") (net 43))
 (segment (start 97.79 96.08) (end 100.87 93) (width 0.25) (layer "B.Cu") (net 43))
 (segment (start 76.08 76.08) (end 77.44 76.08) (width 0.25) (layer "B.Cu") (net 43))
 (segment (start 112.08 96.08) (end 118.11 96.08) (width 0.25) (layer "B.Cu") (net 43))
 (segment (start 88 54) (end 95.91 54) (width 0.25) (layer "B.Cu") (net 43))
 (segment (start 75.08 96.08) (end 77.47 96.08) (width 0.25) (layer "B.Cu") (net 43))
 (segment (start 95.91 54) (end 97.79 55.88) (width 0.25) (layer "B.Cu") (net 43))
 (segment (start 90 78.605536) (end 95.22 73.385536) (width 0.25) (layer "F.Cu") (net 25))
 (segment (start 90 99) (end 90 78.605536) (width 0.25) (layer "F.Cu") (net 25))
 (segment (start 95.22 73.385536) (end 95.22 68.58) (width 0.25) (layer "F.Cu") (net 25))
 (segment (start 101.824465 68.205535) (end 101.824465 81.064465) (width 0.25) (layer "B.Cu") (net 26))
 (segment (start 101.69 65.92) (end 101.57 66.04) (width 0.25) (layer "B.Cu") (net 26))
 (segment (start 101.824465 81.064465) (end 104.14 83.38) (width 0.25) (layer "B.Cu") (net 26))
 (segment (start 104.11 65.92) (end 101.824465 68.205535) (width 0.25) (layer "B.Cu") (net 26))
 (segment (start 104.11 65.92) (end 101.69 65.92) (width 0.25) (layer "B.Cu") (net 26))
 (segment (start 104.14 85.92) (end 101.6 85.92) (width 0.25) (layer "B.Cu") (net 6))
 (segment (start 128 94) (end 128 52) (width 0.25) (layer "F.Cu") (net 21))
 (segment (start 94 99) (end 95 100) (width 0.25) (layer "F.Cu") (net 21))
 (segment (start 95 100) (end 122 100) (width 0.25) (layer "F.Cu") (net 21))
 (segment (start 128 52) (end 124.26 48.26) (width 0.25) (layer "F.Cu") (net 21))
 (segment (start 124.26 48.26) (end 115.57 48.26) (width 0.25) (layer "F.Cu") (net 21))
 (segment (start 122 100) (end 128 94) (width 0.25) (layer "F.Cu") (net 21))
 (segment (start 124.43 65.92) (end 122.144465 68.205535) (width 0.25) (layer "B.Cu") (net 38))
 (segment (start 122.144465 81.064465) (end 124.46 83.38) (width 0.25) (layer "B.Cu") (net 38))
 (segment (start 122.144465 68.205535) (end 122.144465 81.064465) (width 0.25) (layer "B.Cu") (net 38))
 (segment (start 124.43 65.92) (end 121.89 65.92) (width 0.25) (layer "B.Cu") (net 38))
 (segment (start 93 94) (end 109 94) (width 0.25) (layer "F.Cu") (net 29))
 (segment (start 92 99) (end 92 95) (width 0.25) (layer "F.Cu") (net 29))
 (segment (start 114.54 88.46) (end 115.57 88.46) (width 0.25) (layer "F.Cu") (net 29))
 (segment (start 92 95) (end 93 94) (width 0.25) (layer "F.Cu") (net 29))
 (segment (start 109 94) (end 114.54 88.46) (width 0.25) (layer "F.Cu") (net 29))
 (segment (start 124.46 85.92) (end 121.92 85.92) (width 0.25) (layer "B.Cu") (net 30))
 (segment (start 101.6 45.72) (end 106.68 50.8) (width 0.25) (layer "B.Cu") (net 14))
 (segment (start 88.9 45.72) (end 101.6 45.72) (width 0.25) (layer "B.Cu") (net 14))
 (segment (start 106.68 50.8) (end 104.11 53.37) (width 0.25) (layer "B.Cu") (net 14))
 (segment (start 104.11 53.37) (end 104.11 63.38) (width 0.25) (layer "B.Cu") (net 14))
 (segment (start 86.36 48.26) (end 88.9 45.72) (width 0.25) (layer "B.Cu") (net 14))
 (segment (start 106.68 48.26) (end 109.22 45.72) (width 0.25) (layer "B.Cu") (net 22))
 (segment (start 121.92 45.72) (end 121.92 54.561987) (width 0.25) (layer "B.Cu") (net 22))
 (segment (start 121.92 54.561987) (end 124.43 57.071987) (width 0.25) (layer "B.Cu") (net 22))
 (segment (start 109.22 45.72) (end 121.92 45.72) (width 0.25) (layer "B.Cu") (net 22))
 (segment (start 124.43 57.071987) (end 124.43 63.38) (width 0.25) (layer "B.Cu") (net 22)))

